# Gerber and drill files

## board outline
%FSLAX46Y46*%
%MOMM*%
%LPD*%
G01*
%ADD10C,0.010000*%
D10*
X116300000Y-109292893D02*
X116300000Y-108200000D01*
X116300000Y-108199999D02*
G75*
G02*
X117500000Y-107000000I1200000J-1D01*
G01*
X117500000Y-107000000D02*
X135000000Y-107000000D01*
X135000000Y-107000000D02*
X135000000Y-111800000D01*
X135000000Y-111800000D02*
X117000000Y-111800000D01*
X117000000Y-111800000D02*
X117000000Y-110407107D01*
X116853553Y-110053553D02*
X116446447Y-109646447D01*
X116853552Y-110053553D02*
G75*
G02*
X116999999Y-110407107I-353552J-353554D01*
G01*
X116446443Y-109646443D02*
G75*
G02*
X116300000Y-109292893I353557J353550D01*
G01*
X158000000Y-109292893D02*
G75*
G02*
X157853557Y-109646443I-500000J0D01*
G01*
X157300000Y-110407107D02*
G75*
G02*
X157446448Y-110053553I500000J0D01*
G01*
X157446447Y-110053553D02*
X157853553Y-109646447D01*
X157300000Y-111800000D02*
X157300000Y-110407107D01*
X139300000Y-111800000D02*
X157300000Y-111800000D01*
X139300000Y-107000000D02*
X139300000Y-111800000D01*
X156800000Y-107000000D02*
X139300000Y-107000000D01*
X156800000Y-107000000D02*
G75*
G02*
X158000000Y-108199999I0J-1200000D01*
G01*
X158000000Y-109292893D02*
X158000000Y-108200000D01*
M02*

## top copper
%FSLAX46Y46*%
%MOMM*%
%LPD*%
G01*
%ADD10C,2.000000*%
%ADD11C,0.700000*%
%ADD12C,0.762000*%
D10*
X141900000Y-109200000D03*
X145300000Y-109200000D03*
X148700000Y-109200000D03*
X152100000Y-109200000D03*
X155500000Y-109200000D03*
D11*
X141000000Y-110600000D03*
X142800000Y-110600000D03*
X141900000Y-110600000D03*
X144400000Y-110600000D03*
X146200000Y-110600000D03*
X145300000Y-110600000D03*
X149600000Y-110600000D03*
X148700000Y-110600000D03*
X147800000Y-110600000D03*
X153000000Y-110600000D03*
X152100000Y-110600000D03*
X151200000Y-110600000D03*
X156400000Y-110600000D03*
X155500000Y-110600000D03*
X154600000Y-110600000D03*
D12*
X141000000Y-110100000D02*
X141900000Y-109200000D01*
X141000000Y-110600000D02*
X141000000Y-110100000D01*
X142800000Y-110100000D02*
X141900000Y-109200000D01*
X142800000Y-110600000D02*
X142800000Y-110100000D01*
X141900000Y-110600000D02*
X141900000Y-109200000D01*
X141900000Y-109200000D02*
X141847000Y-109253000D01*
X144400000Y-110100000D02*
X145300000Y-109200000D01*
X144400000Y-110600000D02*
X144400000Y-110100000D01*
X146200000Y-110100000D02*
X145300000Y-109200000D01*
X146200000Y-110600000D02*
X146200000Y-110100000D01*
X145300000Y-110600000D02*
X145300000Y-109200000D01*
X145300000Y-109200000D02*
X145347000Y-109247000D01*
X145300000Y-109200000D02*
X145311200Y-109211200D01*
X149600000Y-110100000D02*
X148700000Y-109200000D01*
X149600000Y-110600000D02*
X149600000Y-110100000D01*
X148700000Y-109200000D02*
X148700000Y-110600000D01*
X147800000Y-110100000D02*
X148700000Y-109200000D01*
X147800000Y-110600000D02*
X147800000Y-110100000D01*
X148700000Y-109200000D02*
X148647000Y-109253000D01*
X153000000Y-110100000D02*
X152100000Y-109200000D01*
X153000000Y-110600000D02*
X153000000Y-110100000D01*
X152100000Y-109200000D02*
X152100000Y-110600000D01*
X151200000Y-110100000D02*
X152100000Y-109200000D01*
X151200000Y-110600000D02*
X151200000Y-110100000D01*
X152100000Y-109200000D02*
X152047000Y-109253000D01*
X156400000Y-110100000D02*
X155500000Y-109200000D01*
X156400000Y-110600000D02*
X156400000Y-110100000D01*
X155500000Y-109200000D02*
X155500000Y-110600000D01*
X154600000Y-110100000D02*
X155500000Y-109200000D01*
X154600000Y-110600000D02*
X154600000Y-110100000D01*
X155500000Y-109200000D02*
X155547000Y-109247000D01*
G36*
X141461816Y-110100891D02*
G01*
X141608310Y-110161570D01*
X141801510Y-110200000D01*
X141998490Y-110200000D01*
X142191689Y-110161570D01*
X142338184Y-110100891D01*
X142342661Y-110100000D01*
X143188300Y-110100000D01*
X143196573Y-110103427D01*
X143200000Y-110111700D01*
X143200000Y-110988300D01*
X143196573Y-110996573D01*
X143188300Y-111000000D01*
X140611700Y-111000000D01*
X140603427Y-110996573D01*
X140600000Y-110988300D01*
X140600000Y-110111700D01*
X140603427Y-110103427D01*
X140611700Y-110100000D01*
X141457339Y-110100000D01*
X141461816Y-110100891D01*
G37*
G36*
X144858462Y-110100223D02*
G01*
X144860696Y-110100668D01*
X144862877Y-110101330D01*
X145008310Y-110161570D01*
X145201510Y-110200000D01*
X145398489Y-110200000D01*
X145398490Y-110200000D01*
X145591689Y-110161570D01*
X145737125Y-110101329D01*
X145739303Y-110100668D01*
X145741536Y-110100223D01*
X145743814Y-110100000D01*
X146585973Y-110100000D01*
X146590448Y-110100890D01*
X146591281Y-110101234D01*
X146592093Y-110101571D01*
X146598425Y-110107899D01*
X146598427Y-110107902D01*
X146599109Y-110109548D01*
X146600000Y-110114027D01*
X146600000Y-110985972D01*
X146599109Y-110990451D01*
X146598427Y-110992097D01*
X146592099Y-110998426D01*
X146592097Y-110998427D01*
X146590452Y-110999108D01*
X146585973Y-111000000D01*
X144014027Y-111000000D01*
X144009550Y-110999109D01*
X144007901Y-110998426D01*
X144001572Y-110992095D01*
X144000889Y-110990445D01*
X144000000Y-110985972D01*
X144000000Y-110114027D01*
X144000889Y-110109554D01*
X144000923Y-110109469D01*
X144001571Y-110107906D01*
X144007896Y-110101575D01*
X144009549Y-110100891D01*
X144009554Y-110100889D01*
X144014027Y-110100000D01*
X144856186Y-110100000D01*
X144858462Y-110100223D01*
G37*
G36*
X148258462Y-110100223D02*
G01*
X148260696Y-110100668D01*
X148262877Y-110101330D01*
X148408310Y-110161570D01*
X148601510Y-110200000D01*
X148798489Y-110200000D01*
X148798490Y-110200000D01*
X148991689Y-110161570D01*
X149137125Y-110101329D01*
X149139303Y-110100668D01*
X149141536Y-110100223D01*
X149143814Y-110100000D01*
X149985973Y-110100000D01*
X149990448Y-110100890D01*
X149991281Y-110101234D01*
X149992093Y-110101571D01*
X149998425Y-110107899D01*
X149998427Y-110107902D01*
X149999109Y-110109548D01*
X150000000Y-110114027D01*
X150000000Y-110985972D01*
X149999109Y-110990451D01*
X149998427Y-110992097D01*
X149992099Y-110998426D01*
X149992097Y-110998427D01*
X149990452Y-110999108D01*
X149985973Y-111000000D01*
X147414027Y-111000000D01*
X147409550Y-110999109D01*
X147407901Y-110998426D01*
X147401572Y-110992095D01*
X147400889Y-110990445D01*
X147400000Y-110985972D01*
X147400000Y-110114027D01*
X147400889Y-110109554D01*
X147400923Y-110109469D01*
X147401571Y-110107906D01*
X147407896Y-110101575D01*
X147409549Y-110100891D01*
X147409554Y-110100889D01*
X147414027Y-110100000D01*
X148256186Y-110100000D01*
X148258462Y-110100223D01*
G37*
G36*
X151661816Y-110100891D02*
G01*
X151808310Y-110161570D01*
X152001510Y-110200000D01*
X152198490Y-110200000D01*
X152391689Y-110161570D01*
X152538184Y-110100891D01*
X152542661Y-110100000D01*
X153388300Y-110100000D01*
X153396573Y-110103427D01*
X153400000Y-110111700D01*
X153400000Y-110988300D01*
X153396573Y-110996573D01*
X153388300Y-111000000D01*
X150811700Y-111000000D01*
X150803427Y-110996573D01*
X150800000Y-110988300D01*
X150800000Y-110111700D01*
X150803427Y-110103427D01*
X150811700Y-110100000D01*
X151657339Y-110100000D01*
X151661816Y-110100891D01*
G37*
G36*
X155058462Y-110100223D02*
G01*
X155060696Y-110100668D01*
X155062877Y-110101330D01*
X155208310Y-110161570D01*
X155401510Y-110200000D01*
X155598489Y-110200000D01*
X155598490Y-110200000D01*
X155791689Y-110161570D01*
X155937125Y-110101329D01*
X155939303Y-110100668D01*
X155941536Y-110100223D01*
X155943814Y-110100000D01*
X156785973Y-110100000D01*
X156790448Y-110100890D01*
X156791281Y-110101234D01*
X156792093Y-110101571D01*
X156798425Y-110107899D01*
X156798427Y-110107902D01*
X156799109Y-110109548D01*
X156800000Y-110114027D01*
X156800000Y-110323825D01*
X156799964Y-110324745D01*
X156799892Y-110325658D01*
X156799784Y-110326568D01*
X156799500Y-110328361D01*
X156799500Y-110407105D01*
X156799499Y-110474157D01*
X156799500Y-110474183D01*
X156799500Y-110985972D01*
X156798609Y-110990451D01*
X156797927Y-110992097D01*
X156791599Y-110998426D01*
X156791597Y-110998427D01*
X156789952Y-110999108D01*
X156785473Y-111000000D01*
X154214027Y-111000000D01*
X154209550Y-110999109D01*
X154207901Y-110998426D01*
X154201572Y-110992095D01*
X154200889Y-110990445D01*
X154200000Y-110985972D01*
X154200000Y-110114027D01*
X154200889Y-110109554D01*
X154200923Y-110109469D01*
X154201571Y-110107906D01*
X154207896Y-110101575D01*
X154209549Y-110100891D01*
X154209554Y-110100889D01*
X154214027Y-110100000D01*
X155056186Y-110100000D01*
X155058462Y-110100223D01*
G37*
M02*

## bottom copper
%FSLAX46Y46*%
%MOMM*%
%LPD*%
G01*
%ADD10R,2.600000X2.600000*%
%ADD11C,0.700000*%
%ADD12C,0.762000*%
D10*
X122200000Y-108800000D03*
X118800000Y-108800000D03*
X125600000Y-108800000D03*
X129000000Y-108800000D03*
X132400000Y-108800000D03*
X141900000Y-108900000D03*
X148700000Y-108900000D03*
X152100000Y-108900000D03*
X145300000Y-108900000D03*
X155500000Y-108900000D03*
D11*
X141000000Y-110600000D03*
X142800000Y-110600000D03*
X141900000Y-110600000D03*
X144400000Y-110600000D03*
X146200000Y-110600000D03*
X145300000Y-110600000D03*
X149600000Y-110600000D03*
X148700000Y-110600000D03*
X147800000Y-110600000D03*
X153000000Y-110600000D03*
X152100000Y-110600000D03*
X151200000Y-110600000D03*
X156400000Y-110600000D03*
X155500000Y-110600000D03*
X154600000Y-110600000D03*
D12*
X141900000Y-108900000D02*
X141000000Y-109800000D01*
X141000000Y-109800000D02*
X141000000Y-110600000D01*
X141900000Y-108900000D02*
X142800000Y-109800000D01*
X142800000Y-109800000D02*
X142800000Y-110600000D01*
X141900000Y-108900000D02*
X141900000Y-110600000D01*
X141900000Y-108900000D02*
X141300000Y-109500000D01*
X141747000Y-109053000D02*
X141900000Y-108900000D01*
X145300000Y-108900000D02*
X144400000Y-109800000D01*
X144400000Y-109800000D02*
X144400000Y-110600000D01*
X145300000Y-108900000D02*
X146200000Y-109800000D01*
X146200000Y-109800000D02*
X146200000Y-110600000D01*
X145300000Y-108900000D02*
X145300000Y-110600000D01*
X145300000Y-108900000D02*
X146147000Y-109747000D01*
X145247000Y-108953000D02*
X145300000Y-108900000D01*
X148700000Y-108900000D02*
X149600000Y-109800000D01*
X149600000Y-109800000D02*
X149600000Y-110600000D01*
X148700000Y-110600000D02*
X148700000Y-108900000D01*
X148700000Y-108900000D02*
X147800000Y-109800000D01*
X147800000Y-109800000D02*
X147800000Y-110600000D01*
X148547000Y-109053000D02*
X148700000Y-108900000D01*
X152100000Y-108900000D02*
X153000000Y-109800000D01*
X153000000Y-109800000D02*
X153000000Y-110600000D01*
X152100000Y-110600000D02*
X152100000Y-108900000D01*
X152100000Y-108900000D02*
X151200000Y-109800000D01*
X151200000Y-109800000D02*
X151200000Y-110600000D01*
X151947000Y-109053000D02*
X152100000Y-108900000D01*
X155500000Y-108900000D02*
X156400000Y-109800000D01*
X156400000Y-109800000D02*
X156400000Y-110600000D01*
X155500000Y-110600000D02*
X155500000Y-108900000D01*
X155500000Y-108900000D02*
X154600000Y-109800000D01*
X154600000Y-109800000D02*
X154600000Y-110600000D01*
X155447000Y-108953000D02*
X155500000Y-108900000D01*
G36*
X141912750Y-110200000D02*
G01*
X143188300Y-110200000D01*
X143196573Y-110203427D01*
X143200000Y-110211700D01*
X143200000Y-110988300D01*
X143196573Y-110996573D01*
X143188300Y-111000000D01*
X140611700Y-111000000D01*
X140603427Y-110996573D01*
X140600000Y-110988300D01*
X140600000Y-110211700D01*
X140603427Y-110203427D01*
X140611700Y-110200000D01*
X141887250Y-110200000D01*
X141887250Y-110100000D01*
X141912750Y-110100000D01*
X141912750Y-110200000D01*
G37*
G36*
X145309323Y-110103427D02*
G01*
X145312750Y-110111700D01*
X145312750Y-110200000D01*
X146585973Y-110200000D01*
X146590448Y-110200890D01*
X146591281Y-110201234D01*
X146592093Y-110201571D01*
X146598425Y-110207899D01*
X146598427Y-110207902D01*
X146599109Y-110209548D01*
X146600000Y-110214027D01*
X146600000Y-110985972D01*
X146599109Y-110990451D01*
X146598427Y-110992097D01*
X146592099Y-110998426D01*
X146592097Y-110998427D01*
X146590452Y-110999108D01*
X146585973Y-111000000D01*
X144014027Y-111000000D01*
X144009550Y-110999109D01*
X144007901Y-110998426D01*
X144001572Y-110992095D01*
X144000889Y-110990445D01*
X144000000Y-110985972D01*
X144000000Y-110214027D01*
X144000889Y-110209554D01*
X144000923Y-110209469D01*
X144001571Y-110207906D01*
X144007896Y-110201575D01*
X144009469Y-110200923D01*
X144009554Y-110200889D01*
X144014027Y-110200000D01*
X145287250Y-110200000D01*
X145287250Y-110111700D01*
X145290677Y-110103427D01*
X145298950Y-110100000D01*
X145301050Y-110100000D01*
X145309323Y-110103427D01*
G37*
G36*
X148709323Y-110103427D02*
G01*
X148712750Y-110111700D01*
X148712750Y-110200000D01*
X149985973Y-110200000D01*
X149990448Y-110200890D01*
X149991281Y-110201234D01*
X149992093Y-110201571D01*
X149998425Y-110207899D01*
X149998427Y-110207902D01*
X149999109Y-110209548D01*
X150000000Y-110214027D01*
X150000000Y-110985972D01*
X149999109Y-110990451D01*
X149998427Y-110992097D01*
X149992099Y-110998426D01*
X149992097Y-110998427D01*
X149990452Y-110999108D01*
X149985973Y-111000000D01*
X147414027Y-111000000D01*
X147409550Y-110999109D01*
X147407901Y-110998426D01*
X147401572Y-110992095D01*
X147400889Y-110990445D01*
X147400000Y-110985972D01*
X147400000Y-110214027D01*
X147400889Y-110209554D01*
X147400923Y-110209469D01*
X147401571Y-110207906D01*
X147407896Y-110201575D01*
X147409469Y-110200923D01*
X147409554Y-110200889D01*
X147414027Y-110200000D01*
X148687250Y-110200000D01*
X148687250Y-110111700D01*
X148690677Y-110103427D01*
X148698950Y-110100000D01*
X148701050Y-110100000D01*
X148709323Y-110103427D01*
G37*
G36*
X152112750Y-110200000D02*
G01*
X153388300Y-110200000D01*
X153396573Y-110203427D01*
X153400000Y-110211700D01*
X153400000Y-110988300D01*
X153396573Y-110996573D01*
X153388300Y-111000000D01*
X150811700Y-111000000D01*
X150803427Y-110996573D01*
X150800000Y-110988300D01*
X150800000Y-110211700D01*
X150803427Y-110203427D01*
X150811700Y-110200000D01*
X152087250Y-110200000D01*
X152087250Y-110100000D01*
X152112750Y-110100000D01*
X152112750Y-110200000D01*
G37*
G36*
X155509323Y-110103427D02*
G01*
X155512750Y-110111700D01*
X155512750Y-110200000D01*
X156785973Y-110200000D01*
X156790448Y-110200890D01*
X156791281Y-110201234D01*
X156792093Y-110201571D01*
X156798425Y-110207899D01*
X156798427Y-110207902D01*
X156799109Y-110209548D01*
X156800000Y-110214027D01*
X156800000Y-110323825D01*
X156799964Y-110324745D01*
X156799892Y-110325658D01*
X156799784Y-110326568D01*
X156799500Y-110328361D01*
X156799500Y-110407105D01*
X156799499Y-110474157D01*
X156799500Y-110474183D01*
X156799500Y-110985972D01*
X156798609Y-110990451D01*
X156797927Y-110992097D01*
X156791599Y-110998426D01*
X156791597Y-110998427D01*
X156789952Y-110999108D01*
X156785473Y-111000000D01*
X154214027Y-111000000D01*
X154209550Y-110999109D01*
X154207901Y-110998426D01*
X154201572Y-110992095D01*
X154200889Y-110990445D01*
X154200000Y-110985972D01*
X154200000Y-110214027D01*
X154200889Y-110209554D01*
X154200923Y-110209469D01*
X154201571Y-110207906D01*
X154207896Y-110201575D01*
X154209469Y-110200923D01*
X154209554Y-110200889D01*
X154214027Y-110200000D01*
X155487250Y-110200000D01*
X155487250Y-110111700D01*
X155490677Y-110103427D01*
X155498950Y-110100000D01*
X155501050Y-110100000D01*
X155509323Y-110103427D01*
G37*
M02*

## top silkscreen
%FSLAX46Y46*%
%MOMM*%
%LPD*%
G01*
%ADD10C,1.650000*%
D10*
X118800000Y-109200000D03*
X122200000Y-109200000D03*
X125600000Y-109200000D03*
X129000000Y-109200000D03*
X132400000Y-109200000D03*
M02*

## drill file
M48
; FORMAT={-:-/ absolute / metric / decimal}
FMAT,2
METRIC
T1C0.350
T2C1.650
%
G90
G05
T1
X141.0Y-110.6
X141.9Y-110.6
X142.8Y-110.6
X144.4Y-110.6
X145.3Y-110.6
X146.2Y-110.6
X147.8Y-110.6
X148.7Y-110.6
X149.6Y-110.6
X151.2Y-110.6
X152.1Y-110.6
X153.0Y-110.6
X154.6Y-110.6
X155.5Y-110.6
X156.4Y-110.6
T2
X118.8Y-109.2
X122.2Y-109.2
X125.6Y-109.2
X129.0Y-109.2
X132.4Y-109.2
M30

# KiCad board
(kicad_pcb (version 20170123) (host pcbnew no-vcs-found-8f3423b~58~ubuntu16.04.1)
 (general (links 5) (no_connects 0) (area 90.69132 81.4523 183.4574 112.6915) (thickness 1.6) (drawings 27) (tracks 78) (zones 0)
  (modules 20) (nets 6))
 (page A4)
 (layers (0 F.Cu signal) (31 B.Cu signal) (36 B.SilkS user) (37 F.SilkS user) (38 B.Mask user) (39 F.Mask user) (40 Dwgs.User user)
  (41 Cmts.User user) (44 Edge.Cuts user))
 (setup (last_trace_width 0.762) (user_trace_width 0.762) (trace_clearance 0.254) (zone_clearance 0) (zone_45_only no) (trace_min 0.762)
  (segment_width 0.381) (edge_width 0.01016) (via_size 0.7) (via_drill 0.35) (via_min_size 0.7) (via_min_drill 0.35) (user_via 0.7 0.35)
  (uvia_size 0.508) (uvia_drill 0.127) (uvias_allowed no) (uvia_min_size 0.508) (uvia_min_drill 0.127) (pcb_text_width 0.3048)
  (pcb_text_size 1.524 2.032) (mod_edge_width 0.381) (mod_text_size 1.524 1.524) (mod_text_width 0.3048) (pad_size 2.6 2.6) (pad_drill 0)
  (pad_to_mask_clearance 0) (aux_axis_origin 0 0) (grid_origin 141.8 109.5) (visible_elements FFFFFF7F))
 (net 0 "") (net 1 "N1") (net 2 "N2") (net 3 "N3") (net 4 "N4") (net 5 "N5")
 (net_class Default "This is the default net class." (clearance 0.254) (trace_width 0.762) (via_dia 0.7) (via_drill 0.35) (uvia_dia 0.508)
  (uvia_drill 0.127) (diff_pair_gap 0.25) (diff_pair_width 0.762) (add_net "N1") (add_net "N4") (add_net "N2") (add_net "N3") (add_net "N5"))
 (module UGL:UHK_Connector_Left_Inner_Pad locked (layer B.Cu) (at 122.2 108.8 180)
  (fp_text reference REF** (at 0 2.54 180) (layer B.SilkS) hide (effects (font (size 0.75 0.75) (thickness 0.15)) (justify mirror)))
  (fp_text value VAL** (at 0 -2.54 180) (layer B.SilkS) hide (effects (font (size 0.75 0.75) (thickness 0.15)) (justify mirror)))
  (pad "" smd rect (at 0 0 180) (size 2.6 2.6) (layers B.Cu B.Mask)))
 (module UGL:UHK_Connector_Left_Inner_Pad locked (layer B.Cu) (at 118.8 109.2 180)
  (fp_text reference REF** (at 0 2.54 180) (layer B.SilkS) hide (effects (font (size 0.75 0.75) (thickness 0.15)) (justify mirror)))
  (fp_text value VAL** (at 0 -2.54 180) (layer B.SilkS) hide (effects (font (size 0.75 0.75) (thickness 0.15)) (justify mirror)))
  (pad "" smd rect (at 0 0.4 180) (size 2.6 2.6) (layers B.Cu B.Mask)))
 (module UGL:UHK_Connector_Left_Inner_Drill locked (layer F.Cu) (at 118.8 109.2)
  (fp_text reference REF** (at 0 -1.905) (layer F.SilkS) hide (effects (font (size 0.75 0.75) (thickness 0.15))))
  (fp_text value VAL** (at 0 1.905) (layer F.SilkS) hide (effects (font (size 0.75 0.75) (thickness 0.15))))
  (pad "" np_thru_hole circle (at 0 0) (size 1.65 1.65) (drill 1.65) (layers *.Cu *.Mask F.SilkS)))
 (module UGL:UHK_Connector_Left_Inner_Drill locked (layer F.Cu) (at 122.2 109.2)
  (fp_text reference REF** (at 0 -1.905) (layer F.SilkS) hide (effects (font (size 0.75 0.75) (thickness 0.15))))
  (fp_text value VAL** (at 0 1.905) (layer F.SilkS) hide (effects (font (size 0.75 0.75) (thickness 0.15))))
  (pad "" np_thru_hole circle (at 0 0) (size 1.65 1.65) (drill 1.65) (layers *.Cu *.Mask F.SilkS)))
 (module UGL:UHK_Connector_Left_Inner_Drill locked (layer F.Cu) (at 125.6 109.2)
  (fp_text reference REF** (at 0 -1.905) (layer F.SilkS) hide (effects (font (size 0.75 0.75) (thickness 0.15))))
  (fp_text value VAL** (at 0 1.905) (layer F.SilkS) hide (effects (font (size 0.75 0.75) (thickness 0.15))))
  (pad "" np_thru_hole circle (at 0 0) (size 1.65 1.65) (drill 1.65) (layers *.Cu *.Mask F.SilkS)))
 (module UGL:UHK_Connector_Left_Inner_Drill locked (layer F.Cu) (at 129 109.2)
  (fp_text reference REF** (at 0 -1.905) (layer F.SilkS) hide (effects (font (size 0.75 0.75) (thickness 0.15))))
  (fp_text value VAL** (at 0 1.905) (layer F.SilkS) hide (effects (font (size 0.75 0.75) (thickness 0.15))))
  (pad "" np_thru_hole circle (at 0 0) (size 1.65 1.65) (drill 1.65) (layers *.Cu *.Mask F.SilkS)))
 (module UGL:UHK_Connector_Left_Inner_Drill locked (layer F.Cu) (at 132.4 109.2)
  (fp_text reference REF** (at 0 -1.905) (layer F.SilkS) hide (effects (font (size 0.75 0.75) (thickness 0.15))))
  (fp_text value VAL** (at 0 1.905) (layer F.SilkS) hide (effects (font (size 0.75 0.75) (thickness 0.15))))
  (pad "" np_thru_hole circle (at 0 0) (size 1.65 1.65) (drill 1.65) (layers *.Cu *.Mask F.SilkS)))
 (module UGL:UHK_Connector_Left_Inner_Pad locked (layer B.Cu) (at 125.6 108.8 180)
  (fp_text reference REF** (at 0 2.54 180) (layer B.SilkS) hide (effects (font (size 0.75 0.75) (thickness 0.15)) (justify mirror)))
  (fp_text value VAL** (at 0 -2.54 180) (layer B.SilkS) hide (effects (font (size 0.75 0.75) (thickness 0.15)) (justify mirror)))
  (pad "" smd rect (at 0 0 180) (size 2.6 2.6) (layers B.Cu B.Mask)))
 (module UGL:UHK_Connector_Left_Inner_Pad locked (layer B.Cu) (at 129 108.8 180)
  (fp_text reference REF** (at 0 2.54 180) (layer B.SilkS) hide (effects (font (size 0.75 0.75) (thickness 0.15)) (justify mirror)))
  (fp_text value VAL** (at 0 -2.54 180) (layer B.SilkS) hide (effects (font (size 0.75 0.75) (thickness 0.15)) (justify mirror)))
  (pad "" smd rect (at 0 0 180) (size 2.6 2.6) (layers B.Cu B.Mask)))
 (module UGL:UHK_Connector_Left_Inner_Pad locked (layer B.Cu) (at 132.4 108.8 180)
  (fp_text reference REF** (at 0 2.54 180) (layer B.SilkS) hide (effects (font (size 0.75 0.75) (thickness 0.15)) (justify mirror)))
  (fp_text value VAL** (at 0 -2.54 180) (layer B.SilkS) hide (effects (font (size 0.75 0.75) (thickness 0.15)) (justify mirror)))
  (pad "" smd rect (at 0 0 180) (size 2.6 2.6) (layers B.Cu B.Mask)))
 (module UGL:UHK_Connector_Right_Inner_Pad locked (layer B.Cu) (at 146.31 108.9)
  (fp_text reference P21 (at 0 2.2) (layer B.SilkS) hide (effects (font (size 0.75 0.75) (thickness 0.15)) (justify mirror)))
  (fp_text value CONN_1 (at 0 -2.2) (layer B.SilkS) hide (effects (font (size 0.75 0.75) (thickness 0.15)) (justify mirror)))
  (pad 1 smd rect (at -4.41 0) (size 2.6 2.6) (layers B.Cu B.Mask) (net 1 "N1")))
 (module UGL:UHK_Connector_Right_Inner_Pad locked (layer B.Cu) (at 151.15 108.9)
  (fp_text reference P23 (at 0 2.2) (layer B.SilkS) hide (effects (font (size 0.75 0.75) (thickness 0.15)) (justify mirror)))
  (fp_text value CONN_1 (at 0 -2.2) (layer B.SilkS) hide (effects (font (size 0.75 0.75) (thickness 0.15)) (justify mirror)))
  (pad 1 smd rect (at -2.45 0) (size 2.6 2.6) (layers B.Cu B.Mask) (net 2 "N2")))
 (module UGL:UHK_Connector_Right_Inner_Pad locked (layer B.Cu) (at 153.57 108.9)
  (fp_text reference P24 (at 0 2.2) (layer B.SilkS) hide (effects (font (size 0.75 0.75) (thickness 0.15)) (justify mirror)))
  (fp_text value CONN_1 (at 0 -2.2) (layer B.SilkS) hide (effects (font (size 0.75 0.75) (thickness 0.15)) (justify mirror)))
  (pad 1 smd rect (at -1.47 0) (size 2.6 2.6) (layers B.Cu B.Mask) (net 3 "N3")))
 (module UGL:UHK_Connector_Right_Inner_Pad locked (layer B.Cu) (at 148.73 108.9)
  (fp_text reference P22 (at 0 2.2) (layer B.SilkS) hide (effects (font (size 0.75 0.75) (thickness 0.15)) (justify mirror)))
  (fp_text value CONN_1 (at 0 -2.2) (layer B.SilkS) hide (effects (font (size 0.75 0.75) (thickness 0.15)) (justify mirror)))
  (pad 1 smd rect (at -3.43 0) (size 2.6 2.6) (layers B.Cu B.Mask) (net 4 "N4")))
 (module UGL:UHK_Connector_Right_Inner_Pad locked (layer B.Cu) (at 155.99 108.9)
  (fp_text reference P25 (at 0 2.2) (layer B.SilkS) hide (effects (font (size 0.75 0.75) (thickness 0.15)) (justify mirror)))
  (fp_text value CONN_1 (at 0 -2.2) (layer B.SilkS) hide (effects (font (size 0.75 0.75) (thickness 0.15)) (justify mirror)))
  (pad 1 smd rect (at -0.49 0) (size 2.6 2.6) (layers B.Cu B.Mask) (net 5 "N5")))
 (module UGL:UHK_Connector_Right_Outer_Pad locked (layer F.Cu) (at 141.9 109.2)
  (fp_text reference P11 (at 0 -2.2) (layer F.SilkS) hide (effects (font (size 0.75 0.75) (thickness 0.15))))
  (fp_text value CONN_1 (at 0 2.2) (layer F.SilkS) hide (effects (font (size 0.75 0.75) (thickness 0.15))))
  (pad 1 smd circle (at 0 0) (size 2 2) (layers F.Cu F.Mask) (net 1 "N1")))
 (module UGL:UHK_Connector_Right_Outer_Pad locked (layer F.Cu) (at 145.3 109.2)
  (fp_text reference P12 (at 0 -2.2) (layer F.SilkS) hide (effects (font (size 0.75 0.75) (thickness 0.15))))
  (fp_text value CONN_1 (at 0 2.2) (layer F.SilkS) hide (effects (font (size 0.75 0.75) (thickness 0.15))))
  (pad 1 smd circle (at 0 0) (size 2 2) (layers F.Cu F.Mask) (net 4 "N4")))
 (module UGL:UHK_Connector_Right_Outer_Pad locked (layer F.Cu) (at 148.7 109.2)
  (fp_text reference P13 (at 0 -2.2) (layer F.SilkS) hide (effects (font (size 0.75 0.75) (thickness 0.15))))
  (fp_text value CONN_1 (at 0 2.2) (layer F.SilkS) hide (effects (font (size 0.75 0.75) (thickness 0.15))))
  (pad 1 smd circle (at 0 0) (size 2 2) (layers F.Cu F.Mask) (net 2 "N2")))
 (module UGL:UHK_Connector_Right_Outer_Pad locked (layer F.Cu) (at 152.1 109.2)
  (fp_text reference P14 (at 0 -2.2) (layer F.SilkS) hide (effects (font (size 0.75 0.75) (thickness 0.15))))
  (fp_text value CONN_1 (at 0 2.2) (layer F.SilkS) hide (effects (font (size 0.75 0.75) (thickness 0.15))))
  (pad 1 smd circle (at 0 0) (size 2 2) (layers F.Cu F.Mask) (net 3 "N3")))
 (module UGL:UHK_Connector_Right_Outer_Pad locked (layer F.Cu) (at 155.5 109.2)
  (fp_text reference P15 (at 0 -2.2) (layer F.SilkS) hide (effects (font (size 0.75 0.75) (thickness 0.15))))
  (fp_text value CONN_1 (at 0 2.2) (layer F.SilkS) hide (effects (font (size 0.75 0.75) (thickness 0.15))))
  (pad 1 smd circle (at 0 0) (size 2 2) (layers F.Cu F.Mask) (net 5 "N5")))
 (gr_line (start 116.3 109.292893) (end 116.3 108.2) (angle 90) (layer Edge.Cuts) (width 0.01))
 (gr_arc (start 117.5 108.2) (end 117.5 107) (angle -89.99995347) (layer Edge.Cuts) (width 0.01))
 (gr_line (start 117.5 107) (end 135 107) (angle 90) (layer Edge.Cuts) (width 0.01))
 (gr_line (start 135 107) (end 135 111.8) (angle 90) (layer Edge.Cuts) (width 0.01))
 (gr_line (start 135 111.8) (end 117 111.8) (angle 90) (layer Edge.Cuts) (width 0.01))
 (gr_line (start 117 111.8) (end 117 110.407107) (angle 90) (layer Edge.Cuts) (width 0.01))
 (gr_line (start 116.853553 110.053553) (end 116.446447 109.646447) (angle 90) (layer Edge.Cuts) (width 0.01))
 (gr_arc (start 116.5 110.407107) (end 117 110.407107) (angle -45.00015451) (layer Edge.Cuts) (width 0.01))
 (gr_arc (start 116.8 109.292893) (end 116.3 109.292893) (angle -44.99944414) (layer Edge.Cuts) (width 0.01))
 (gr_arc (start 157.5 109.292893) (end 158 109.292893) (angle 44.99944414) (layer Edge.Cuts) (width 0.01))
 (gr_arc (start 157.8 110.407107) (end 157.3 110.407107) (angle 45.00015451) (layer Edge.Cuts) (width 0.01))
 (gr_line (start 157.446447 110.053553) (end 157.853553 109.646447) (angle 90) (layer Edge.Cuts) (width 0.01))
 (gr_line (start 157.3 111.8) (end 157.3 110.407107) (angle 90) (layer Edge.Cuts) (width 0.01))
 (gr_line (start 139.3 111.8) (end 157.3 111.8) (angle 90) (layer Edge.Cuts) (width 0.01))
 (gr_line (start 139.3 107) (end 139.3 111.8) (angle 90) (layer Edge.Cuts) (width 0.01))
 (gr_line (start 156.8 107) (end 139.3 107) (angle 90) (layer Edge.Cuts) (width 0.01))
 (gr_arc (start 156.8 108.2) (end 156.8 107) (angle 89.99995347) (layer Edge.Cuts) (width 0.01))
 (gr_line (start 158 109.292893) (end 158 108.2) (angle 90) (layer Edge.Cuts) (width 0.01))
 (segment (start 141.9 108.9) (end 141 109.8) (width 0.762) (layer B.Cu) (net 1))
 (segment (start 141 109.8) (end 141 110.6) (width 0.762) (layer B.Cu) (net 1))
 (segment (start 141 110.1) (end 141.9 109.2) (width 0.762) (layer F.Cu) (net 1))
 (segment (start 141 110.6) (end 141 110.1) (width 0.762) (layer F.Cu) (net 1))
 (via (at 141 110.6) (size 0.7) (drill 0.35) (layers F.Cu B.Cu) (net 1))
 (segment (start 141.9 108.9) (end 142.8 109.8) (width 0.762) (layer B.Cu) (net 1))
 (segment (start 142.8 109.8) (end 142.8 110.6) (width 0.762) (layer B.Cu) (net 1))
 (segment (start 142.8 110.1) (end 141.9 109.2) (width 0.762) (layer F.Cu) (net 1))
 (segment (start 142.8 110.6) (end 142.8 110.1) (width 0.762) (layer F.Cu) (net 1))
 (via (at 142.8 110.6) (size 0.7) (drill 0.35) (layers F.Cu B.Cu) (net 1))
 (segment (start 141.9 108.9) (end 141.9 110.6) (width 0.762) (layer B.Cu) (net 1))
 (segment (start 141.9 110.6) (end 141.9 109.2) (width 0.762) (layer F.Cu) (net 1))
 (via (at 141.9 110.6) (size 0.7) (drill 0.35) (layers F.Cu B.Cu) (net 1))
 (segment (start 141.9 108.9) (end 141.3 109.5) (width 0.762) (layer B.Cu) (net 1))
 (segment (start 141.9 109.2) (end 141.847 109.253) (width 0.762) (layer F.Cu) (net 1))
 (segment (start 141.747 109.053) (end 141.9 108.9) (width 0.762) (layer B.Cu) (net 1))
 (segment (start 145.3 108.9) (end 144.4 109.8) (width 0.762) (layer B.Cu) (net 4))
 (segment (start 144.4 109.8) (end 144.4 110.6) (width 0.762) (layer B.Cu) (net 4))
 (segment (start 144.4 110.1) (end 145.3 109.2) (width 0.762) (layer F.Cu) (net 4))
 (segment (start 144.4 110.6) (end 144.4 110.1) (width 0.762) (layer F.Cu) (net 4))
 (via (at 144.4 110.6) (size 0.7) (drill 0.35) (layers F.Cu B.Cu) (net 4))
 (segment (start 145.3 108.9) (end 146.2 109.8) (width 0.762) (layer B.Cu) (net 4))
 (segment (start 146.2 109.8) (end 146.2 110.6) (width 0.762) (layer B.Cu) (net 4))
 (segment (start 146.2 110.1) (end 145.3 109.2) (width 0.762) (layer F.Cu) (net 4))
 (segment (start 146.2 110.6) (end 146.2 110.1) (width 0.762) (layer F.Cu) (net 4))
 (via (at 146.2 110.6) (size 0.7) (drill 0.35) (layers F.Cu B.Cu) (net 4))
 (segment (start 145.3 108.9) (end 145.3 110.6) (width 0.762) (layer B.Cu) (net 4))
 (segment (start 145.3 110.6) (end 145.3 109.2) (width 0.762) (layer F.Cu) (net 4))
 (via (at 145.3 110.6) (size 0.7) (drill 0.35) (layers F.Cu B.Cu) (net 4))
 (segment (start 145.3 108.9) (end 146.147 109.747) (width 0.762) (layer B.Cu) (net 4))
 (segment (start 145.3 109.2) (end 145.347 109.247) (width 0.762) (layer F.Cu) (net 4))
 (segment (start 145.247 108.953) (end 145.3 108.9) (width 0.762) (layer B.Cu) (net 4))
 (segment (start 145.3 109.2) (end 145.3112 109.2112) (width 0.762) (layer F.Cu) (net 4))
 (segment (start 148.7 108.9) (end 149.6 109.8) (width 0.762) (layer B.Cu) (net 2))
 (segment (start 149.6 109.8) (end 149.6 110.6) (width 0.762) (layer B.Cu) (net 2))
 (segment (start 149.6 110.1) (end 148.7 109.2) (width 0.762) (layer F.Cu) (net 2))
 (segment (start 149.6 110.6) (end 149.6 110.1) (width 0.762) (layer F.Cu) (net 2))
 (via (at 149.6 110.6) (size 0.7) (drill 0.35) (layers F.Cu B.Cu) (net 2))
 (segment (start 148.7 109.2) (end 148.7 110.6) (width 0.762) (layer F.Cu) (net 2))
 (segment (start 148.7 110.6) (end 148.7 108.9) (width 0.762) (layer B.Cu) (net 2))
 (via (at 148.7 110.6) (size 0.7) (drill 0.35) (layers F.Cu B.Cu) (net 2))
 (segment (start 148.7 108.9) (end 147.8 109.8) (width 0.762) (layer B.Cu) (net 2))
 (segment (start 147.8 109.8) (end 147.8 110.6) (width 0.762) (layer B.Cu) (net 2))
 (segment (start 147.8 110.1) (end 148.7 109.2) (width 0.762) (layer F.Cu) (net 2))
 (segment (start 147.8 110.6) (end 147.8 110.1) (width 0.762) (layer F.Cu) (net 2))
 (via (at 147.8 110.6) (size 0.7) (drill 0.35) (layers F.Cu B.Cu) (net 2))
 (segment (start 148.7 109.2) (end 148.647 109.253) (width 0.762) (layer F.Cu) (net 2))
 (segment (start 148.547 109.053) (end 148.7 108.9) (width 0.762) (layer B.Cu) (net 2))
 (segment (start 152.1 108.9) (end 153 109.8) (width 0.762) (layer B.Cu) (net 3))
 (segment (start 153 109.8) (end 153 110.6) (width 0.762) (layer B.Cu) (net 3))
 (segment (start 153 110.1) (end 152.1 109.2) (width 0.762) (layer F.Cu) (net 3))
 (segment (start 153 110.6) (end 153 110.1) (width 0.762) (layer F.Cu) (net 3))
 (via (at 153 110.6) (size 0.7) (drill 0.35) (layers F.Cu B.Cu) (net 3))
 (segment (start 152.1 109.2) (end 152.1 110.6) (width 0.762) (layer F.Cu) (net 3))
 (segment (start 152.1 110.6) (end 152.1 108.9) (width 0.762) (layer B.Cu) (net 3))
 (via (at 152.1 110.6) (size 0.7) (drill 0.35) (layers F.Cu B.Cu) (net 3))
 (segment (start 152.1 108.9) (end 151.2 109.8) (width 0.762) (layer B.Cu) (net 3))
 (segment (start 151.2 109.8) (end 151.2 110.6) (width 0.762) (layer B.Cu) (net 3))
 (segment (start 151.2 110.1) (end 152.1 109.2) (width 0.762) (layer F.Cu) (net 3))
 (segment (start 151.2 110.6) (end 151.2 110.1) (width 0.762) (layer F.Cu) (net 3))
 (via (at 151.2 110.6) (size 0.7) (drill 0.35) (layers F.Cu B.Cu) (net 3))
 (segment (start 152.1 109.2) (end 152.047 109.253) (width 0.762) (layer F.Cu) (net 3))
 (segment (start 151.947 109.053) (end 152.1 108.9) (width 0.762) (layer B.Cu) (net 3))
 (segment (start 155.5 108.9) (end 156.4 109.8) (width 0.762) (layer B.Cu) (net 5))
 (segment (start 156.4 109.8) (end 156.4 110.6) (width 0.762) (layer B.Cu) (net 5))
 (segment (start 156.4 110.1) (end 155.5 109.2) (width 0.762) (layer F.Cu) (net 5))
 (segment (start 156.4 110.6) (end 156.4 110.1) (width 0.762) (layer F.Cu) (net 5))
 (via (at 156.4 110.6) (size 0.7) (drill 0.35) (layers F.Cu B.Cu) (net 5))
 (segment (start 155.5 109.2) (end 155.5 110.6) (width 0.762) (layer F.Cu) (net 5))
 (segment (start 155.5 110.6) (end 155.5 108.9) (width 0.762) (layer B.Cu) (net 5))
 (via (at 155.5 110.6) (size 0.7) (drill 0.35) (layers F.Cu B.Cu) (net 5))
 (segment (start 155.5 108.9) (end 154.6 109.8) (width 0.762) (layer B.Cu) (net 5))
 (segment (start 154.6 109.8) (end 154.6 110.6) (width 0.762) (layer B.Cu) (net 5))
 (segment (start 154.6 110.1) (end 155.5 109.2) (width 0.762) (layer F.Cu) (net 5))
 (segment (start 154.6 110.6) (end 154.6 110.1) (width 0.762) (layer F.Cu) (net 5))
 (via (at 154.6 110.6) (size 0.7) (drill 0.35) (layers F.Cu B.Cu) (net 5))
 (segment (start 155.5 109.2) (end 155.547 109.247) (width 0.762) (layer F.Cu) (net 5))
 (segment (start 155.447 108.953) (end 155.5 108.9) (width 0.762) (layer B.Cu) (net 5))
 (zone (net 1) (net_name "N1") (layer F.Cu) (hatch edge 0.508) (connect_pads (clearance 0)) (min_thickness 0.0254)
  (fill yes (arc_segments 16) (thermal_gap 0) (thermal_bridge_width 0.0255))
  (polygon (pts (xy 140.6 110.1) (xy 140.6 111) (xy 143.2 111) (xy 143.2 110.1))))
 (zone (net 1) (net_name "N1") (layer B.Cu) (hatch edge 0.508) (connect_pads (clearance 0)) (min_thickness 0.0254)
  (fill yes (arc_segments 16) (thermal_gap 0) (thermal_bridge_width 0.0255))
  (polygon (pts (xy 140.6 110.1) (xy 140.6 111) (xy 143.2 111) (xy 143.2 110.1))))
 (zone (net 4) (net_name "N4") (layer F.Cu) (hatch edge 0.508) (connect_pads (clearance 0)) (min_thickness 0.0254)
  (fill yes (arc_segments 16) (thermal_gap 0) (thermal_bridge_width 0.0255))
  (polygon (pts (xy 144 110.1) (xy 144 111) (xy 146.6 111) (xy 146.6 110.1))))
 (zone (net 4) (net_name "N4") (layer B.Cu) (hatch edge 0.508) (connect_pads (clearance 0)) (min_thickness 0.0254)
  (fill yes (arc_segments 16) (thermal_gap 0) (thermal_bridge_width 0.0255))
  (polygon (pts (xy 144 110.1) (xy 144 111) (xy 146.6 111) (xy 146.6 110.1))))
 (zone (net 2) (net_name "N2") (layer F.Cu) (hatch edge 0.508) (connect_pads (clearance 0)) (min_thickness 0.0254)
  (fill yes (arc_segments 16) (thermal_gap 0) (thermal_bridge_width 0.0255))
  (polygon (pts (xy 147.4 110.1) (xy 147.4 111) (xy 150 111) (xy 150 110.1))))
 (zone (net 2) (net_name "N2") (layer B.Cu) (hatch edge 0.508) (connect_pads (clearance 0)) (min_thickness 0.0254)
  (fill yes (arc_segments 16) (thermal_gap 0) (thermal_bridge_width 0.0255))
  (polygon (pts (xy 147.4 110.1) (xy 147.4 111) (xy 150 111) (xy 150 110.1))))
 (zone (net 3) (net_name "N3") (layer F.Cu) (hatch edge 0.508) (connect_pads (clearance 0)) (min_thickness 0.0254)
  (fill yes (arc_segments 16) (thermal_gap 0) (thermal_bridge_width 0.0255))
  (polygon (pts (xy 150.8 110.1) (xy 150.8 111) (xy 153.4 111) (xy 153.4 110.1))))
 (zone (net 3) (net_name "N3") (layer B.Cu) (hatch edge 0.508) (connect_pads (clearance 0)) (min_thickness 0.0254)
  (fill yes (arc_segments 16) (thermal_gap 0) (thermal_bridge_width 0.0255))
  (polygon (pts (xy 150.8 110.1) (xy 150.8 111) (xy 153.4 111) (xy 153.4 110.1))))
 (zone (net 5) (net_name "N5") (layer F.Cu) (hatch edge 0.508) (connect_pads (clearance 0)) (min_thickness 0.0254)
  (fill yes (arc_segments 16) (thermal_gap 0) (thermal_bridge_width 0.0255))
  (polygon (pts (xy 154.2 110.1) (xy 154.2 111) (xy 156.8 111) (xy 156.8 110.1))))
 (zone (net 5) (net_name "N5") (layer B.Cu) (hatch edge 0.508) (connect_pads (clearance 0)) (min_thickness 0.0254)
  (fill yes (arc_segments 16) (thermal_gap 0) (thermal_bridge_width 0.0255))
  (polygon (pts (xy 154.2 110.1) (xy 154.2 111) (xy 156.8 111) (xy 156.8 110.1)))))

